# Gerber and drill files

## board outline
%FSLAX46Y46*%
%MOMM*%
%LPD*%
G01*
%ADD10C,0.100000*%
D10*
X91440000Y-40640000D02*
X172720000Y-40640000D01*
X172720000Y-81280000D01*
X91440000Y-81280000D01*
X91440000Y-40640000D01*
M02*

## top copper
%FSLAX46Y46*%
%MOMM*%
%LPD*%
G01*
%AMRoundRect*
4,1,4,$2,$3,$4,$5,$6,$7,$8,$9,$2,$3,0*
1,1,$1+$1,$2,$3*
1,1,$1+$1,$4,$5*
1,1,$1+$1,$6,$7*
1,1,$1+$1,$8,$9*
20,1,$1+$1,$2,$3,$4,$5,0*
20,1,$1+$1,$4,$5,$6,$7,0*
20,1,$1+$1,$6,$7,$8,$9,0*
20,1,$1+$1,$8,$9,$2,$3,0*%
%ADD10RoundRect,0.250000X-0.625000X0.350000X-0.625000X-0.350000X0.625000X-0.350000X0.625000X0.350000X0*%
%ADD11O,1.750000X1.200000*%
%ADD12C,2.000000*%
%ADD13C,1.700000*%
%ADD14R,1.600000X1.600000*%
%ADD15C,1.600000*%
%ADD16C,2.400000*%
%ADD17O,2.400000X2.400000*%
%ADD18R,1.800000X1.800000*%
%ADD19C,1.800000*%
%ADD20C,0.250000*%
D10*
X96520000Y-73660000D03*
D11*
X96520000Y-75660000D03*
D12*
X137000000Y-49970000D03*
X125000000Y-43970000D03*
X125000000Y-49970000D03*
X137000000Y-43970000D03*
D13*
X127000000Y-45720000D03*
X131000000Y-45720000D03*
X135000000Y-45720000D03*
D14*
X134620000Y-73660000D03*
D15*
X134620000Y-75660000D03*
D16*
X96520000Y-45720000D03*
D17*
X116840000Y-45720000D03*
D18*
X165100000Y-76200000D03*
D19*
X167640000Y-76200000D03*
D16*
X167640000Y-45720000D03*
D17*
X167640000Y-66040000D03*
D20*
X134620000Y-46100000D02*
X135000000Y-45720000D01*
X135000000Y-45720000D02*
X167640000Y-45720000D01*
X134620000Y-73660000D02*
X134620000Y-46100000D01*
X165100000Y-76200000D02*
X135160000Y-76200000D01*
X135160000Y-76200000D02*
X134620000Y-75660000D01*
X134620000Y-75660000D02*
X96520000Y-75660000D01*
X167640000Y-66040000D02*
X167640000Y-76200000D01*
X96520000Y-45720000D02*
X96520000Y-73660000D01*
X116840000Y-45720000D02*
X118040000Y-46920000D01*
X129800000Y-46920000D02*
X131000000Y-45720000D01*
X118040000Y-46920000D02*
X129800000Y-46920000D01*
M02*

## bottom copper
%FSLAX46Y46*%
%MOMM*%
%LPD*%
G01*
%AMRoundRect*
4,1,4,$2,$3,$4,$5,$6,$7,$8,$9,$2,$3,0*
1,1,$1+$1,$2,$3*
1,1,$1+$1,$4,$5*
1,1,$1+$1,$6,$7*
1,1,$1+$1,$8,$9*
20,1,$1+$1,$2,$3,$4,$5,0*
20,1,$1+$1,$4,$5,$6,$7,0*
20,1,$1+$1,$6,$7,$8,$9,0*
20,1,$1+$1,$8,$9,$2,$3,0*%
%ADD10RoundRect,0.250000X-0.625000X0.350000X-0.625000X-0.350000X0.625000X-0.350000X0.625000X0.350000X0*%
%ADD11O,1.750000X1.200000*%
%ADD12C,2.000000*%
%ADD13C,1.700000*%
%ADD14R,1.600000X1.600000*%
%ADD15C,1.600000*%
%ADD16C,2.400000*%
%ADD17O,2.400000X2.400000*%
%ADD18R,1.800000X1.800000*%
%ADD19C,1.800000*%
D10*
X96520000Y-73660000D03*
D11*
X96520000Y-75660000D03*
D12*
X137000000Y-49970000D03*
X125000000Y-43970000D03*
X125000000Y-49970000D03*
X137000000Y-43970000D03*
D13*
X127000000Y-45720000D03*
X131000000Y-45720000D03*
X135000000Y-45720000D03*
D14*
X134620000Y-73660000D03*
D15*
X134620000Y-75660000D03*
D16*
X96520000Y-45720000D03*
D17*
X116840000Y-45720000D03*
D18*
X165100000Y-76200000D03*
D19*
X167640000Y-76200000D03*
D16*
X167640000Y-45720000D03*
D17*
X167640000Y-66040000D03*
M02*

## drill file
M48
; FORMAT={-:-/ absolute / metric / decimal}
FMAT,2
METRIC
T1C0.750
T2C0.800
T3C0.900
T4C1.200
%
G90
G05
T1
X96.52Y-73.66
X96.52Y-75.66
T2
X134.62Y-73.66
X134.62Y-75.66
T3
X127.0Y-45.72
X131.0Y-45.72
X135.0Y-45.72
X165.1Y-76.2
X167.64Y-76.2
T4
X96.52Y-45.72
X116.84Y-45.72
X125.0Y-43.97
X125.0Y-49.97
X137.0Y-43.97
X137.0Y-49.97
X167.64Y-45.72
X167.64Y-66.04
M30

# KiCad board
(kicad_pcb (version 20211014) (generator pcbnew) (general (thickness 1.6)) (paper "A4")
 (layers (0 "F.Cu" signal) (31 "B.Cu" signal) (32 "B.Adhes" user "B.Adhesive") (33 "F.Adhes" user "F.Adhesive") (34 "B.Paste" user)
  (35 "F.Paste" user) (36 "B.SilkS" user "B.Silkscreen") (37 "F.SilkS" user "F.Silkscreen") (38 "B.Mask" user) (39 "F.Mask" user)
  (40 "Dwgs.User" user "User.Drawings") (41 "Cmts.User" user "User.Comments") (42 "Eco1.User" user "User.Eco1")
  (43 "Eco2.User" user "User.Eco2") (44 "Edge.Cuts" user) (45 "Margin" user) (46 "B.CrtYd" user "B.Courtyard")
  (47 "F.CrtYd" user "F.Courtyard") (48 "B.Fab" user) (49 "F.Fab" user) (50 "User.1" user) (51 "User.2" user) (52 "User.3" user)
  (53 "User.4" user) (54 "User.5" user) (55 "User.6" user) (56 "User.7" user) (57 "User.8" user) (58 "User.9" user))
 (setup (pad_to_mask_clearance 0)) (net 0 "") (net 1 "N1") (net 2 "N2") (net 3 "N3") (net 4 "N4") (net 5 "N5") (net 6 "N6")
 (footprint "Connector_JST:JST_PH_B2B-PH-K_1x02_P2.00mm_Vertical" (layer "F.Cu") (at 96.52 73.66 -90)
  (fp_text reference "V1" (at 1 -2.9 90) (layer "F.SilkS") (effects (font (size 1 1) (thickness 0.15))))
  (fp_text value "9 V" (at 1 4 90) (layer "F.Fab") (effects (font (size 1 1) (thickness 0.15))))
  (pad "1" thru_hole roundrect (at 0 0 270) (size 1.2 1.75) (drill 0.75) (layers *.Cu *.Mask) (roundrect_rratio 0.208333) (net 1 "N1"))
  (pad "2" thru_hole oval (at 2 0 270) (size 1.2 1.75) (drill 0.75) (layers *.Cu *.Mask) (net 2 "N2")))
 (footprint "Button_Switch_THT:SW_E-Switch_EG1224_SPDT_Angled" (layer "F.Cu") (at 127 45.72)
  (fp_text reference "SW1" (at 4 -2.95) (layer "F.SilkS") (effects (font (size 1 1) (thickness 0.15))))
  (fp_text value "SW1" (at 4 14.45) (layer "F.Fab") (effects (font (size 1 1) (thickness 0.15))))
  (pad "" thru_hole circle (at 10 4.25) (size 2 2) (drill 1.2) (layers *.Cu *.Mask))
  (pad "" thru_hole circle (at -2 -1.75) (size 2 2) (drill 1.2) (layers *.Cu *.Mask))
  (pad "" thru_hole circle (at -2 4.25) (size 2 2) (drill 1.2) (layers *.Cu *.Mask))
  (pad "" thru_hole circle (at 10 -1.75) (size 2 2) (drill 1.2) (layers *.Cu *.Mask))
  (pad "1" thru_hole circle (at 0 0) (size 1.7 1.7) (drill 0.9) (layers *.Cu *.Mask) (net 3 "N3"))
  (pad "2" thru_hole circle (at 4 0) (size 1.7 1.7) (drill 0.9) (layers *.Cu *.Mask) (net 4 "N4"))
  (pad "3" thru_hole circle (at 8 0) (size 1.7 1.7) (drill 0.9) (layers *.Cu *.Mask) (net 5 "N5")))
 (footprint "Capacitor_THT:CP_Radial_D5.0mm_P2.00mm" (layer "F.Cu") (at 134.62 73.66 -90)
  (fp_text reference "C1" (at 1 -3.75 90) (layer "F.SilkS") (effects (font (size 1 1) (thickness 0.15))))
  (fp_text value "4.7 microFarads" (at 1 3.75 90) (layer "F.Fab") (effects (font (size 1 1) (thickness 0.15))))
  (pad "1" thru_hole rect (at 0 0 270) (size 1.6 1.6) (drill 0.8) (layers *.Cu *.Mask) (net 5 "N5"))
  (pad "2" thru_hole circle (at 2 0 270) (size 1.6 1.6) (drill 0.8) (layers *.Cu *.Mask) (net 2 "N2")))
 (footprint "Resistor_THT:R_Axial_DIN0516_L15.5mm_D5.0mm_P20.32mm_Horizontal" (layer "F.Cu") (at 96.52 45.72)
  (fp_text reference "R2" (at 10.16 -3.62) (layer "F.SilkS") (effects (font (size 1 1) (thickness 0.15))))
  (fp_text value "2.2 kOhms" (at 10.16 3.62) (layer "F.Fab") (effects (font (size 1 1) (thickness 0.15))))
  (pad "1" thru_hole circle (at 0 0) (size 2.4 2.4) (drill 1.2) (layers *.Cu *.Mask) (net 1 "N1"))
  (pad "2" thru_hole oval (at 20.32 0) (size 2.4 2.4) (drill 1.2) (layers *.Cu *.Mask) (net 4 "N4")))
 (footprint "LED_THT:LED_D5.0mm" (layer "F.Cu") (at 165.1 76.2)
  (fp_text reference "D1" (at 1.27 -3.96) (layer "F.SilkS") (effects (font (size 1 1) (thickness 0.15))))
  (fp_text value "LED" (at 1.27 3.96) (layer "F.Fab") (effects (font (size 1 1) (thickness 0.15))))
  (pad "1" thru_hole rect (at 0 0) (size 1.8 1.8) (drill 0.9) (layers *.Cu *.Mask) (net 2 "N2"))
  (pad "2" thru_hole circle (at 2.54 0) (size 1.8 1.8) (drill 0.9) (layers *.Cu *.Mask) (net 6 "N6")))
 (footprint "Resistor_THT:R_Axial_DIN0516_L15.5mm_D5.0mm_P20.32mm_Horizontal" (layer "F.Cu") (at 167.64 45.72 -90)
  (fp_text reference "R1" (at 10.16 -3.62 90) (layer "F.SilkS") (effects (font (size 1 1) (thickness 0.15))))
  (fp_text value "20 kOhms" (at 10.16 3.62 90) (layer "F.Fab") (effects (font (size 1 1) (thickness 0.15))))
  (pad "1" thru_hole circle (at 0 0 270) (size 2.4 2.4) (drill 1.2) (layers *.Cu *.Mask) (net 5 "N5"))
  (pad "2" thru_hole oval (at 20.32 0 270) (size 2.4 2.4) (drill 1.2) (layers *.Cu *.Mask) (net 6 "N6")))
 (gr_rect (start 91.44 40.64) (end 172.72 81.28) (layer "Edge.Cuts") (width 0.1) (fill none))
 (segment (start 134.62 46.1) (end 135 45.72) (width 0.25) (layer "F.Cu") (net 5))
 (segment (start 135 45.72) (end 167.64 45.72) (width 0.25) (layer "F.Cu") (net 5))
 (segment (start 134.62 73.66) (end 134.62 46.1) (width 0.25) (layer "F.Cu") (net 5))
 (segment (start 165.1 76.2) (end 135.16 76.2) (width 0.25) (layer "F.Cu") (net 2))
 (segment (start 135.16 76.2) (end 134.62 75.66) (width 0.25) (layer "F.Cu") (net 2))
 (segment (start 134.62 75.66) (end 96.52 75.66) (width 0.25) (layer "F.Cu") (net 2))
 (segment (start 167.64 66.04) (end 167.64 76.2) (width 0.25) (layer "F.Cu") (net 6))
 (segment (start 96.52 45.72) (end 96.52 73.66) (width 0.25) (layer "F.Cu") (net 1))
 (segment (start 116.84 45.72) (end 118.04 46.92) (width 0.25) (layer "F.Cu") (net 4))
 (segment (start 129.8 46.92) (end 131 45.72) (width 0.25) (layer "F.Cu") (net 4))
 (segment (start 118.04 46.92) (end 129.8 46.92) (width 0.25) (layer "F.Cu") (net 4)))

